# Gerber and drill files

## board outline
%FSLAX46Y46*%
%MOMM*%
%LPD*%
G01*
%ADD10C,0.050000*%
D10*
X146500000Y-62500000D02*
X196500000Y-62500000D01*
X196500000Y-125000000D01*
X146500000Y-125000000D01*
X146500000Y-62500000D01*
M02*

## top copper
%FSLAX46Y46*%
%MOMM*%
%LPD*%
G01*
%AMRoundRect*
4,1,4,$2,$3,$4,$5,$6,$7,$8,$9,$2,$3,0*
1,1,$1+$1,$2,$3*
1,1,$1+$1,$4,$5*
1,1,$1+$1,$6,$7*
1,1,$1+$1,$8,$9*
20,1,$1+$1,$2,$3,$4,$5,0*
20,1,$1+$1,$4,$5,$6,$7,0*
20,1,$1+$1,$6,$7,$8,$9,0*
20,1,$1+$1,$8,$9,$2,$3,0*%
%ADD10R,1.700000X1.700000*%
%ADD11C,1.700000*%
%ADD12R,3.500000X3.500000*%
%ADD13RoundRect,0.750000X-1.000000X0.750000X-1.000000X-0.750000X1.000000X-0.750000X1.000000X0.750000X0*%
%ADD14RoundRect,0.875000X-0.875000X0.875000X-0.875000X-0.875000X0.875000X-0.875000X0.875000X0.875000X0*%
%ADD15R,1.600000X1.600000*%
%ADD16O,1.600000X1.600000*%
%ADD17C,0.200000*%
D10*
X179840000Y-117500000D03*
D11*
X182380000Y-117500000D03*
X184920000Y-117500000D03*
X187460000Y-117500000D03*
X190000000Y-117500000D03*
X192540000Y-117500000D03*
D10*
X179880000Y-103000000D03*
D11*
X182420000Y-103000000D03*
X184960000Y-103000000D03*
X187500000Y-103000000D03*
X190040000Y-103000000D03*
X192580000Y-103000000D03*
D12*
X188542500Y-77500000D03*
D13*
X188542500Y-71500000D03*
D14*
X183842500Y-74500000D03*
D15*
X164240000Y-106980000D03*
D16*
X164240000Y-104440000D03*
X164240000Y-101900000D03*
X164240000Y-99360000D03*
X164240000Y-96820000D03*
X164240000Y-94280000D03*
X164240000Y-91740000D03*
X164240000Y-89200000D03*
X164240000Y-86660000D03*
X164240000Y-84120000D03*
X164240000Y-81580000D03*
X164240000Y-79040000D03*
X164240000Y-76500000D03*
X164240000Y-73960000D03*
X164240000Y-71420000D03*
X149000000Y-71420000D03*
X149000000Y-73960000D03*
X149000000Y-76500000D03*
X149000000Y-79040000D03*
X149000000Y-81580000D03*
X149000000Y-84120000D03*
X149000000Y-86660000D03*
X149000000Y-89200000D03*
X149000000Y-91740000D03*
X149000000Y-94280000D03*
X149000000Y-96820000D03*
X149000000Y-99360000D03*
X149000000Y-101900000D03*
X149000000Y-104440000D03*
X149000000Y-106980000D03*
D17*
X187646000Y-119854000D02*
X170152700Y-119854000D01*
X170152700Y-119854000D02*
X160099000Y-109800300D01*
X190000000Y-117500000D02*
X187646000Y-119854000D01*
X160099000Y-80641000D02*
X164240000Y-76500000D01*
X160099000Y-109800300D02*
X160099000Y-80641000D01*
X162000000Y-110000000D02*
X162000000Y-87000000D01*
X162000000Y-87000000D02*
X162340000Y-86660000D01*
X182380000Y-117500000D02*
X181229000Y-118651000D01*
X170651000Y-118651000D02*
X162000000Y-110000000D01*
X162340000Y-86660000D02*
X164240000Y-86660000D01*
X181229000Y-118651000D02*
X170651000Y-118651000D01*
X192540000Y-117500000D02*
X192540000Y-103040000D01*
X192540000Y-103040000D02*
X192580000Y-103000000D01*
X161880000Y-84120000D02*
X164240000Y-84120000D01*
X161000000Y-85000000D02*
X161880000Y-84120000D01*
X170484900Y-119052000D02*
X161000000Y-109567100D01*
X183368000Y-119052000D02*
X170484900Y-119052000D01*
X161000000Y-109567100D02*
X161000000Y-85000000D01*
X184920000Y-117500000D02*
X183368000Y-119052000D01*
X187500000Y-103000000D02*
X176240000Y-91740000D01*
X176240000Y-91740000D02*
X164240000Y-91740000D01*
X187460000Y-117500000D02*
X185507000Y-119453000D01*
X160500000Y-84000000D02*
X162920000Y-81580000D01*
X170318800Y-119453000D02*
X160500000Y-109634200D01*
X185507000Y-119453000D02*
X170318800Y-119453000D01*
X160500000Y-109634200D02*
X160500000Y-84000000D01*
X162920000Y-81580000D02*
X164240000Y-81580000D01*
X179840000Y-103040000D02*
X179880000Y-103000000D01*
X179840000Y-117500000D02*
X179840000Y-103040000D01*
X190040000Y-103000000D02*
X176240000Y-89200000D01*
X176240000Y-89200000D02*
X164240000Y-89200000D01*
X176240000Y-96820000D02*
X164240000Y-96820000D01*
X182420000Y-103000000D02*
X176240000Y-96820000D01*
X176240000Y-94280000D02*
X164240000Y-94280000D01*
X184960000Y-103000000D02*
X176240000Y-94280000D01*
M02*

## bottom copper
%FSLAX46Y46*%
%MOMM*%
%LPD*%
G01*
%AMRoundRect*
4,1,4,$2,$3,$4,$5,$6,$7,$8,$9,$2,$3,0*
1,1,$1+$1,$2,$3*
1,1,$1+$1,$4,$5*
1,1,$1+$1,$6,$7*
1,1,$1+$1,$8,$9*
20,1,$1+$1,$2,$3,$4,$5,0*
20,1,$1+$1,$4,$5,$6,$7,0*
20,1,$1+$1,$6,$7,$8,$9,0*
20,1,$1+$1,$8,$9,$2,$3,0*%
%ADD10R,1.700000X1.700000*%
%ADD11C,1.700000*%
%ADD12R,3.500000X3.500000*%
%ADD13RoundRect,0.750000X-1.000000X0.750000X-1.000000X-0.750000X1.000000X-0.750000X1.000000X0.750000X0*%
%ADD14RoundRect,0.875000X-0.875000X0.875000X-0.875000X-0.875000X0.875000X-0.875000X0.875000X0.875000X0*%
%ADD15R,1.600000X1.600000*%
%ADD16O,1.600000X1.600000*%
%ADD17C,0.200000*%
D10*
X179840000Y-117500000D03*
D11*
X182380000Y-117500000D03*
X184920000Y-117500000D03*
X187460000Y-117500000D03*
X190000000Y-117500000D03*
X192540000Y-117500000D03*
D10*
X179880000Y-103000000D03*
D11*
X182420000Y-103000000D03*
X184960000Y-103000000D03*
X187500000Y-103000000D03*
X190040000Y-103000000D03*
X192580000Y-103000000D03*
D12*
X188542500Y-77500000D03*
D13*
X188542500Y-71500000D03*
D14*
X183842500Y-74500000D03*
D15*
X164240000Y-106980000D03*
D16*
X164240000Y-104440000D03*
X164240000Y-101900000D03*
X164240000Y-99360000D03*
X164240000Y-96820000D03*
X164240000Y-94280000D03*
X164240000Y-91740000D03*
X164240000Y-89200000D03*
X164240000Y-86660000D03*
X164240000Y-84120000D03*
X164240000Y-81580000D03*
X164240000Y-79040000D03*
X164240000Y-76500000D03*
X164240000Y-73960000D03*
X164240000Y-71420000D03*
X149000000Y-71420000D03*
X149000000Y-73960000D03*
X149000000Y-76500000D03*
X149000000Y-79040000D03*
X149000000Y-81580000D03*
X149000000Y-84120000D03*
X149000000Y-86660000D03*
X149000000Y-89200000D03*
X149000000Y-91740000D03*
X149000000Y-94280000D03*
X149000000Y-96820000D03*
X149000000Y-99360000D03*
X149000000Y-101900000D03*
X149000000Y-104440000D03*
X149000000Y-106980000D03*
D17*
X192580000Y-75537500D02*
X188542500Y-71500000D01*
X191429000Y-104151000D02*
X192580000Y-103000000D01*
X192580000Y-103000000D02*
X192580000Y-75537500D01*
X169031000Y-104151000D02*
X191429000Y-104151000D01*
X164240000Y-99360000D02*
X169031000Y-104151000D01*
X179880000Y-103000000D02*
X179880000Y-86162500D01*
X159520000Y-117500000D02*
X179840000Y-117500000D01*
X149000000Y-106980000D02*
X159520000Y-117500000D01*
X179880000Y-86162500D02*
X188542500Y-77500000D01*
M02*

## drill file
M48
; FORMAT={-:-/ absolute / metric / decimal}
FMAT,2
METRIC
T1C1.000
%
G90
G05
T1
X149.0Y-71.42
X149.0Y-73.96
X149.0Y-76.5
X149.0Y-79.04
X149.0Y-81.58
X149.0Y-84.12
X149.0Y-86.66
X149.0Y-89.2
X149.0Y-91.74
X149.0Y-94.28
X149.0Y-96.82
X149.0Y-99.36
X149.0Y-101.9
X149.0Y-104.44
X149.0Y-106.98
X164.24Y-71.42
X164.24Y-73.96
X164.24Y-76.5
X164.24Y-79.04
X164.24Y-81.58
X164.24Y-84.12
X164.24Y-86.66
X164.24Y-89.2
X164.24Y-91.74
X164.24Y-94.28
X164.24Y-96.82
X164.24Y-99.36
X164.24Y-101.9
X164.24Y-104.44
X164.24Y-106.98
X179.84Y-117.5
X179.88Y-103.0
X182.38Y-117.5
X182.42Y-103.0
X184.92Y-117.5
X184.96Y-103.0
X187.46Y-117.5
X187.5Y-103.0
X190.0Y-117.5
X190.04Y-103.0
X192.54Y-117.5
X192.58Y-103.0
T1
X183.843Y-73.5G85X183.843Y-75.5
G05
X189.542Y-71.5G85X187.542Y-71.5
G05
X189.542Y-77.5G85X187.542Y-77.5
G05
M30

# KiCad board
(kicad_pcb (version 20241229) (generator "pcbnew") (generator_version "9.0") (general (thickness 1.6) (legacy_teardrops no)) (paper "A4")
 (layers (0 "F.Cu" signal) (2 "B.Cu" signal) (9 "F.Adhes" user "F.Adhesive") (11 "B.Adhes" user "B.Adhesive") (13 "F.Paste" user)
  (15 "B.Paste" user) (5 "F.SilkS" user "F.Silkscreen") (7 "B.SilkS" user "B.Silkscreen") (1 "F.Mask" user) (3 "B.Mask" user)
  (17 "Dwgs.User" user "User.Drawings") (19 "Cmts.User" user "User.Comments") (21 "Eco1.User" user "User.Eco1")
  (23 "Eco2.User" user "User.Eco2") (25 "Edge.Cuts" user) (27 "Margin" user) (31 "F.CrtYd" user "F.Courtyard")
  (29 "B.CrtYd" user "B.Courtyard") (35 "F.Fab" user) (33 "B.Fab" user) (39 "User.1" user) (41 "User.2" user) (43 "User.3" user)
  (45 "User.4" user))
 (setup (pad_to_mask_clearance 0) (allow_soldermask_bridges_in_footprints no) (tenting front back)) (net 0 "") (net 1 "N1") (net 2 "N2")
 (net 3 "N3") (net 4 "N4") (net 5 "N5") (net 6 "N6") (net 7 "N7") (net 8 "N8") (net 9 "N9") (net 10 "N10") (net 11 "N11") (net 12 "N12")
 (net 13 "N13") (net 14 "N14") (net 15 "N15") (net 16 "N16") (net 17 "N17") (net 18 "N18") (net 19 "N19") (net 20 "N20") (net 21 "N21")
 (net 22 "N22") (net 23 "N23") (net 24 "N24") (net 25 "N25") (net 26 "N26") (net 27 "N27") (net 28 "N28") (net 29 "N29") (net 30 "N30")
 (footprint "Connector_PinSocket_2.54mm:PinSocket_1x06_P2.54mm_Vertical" (layer "F.Cu") (at 179.84 117.5 90)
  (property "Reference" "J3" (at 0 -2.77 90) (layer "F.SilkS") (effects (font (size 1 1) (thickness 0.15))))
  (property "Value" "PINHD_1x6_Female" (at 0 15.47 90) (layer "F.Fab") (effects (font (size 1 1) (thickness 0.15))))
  (pad "1" thru_hole rect (at 0 0 90) (size 1.7 1.7) (drill 1) (layers "*.Cu" "*.Mask") (remove_unused_layers no) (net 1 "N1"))
  (pad "2" thru_hole circle (at 0 2.54 90) (size 1.7 1.7) (drill 1) (layers "*.Cu" "*.Mask") (remove_unused_layers no) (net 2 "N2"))
  (pad "3" thru_hole circle (at 0 5.08 90) (size 1.7 1.7) (drill 1) (layers "*.Cu" "*.Mask") (remove_unused_layers no) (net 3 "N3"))
  (pad "4" thru_hole circle (at 0 7.62 90) (size 1.7 1.7) (drill 1) (layers "*.Cu" "*.Mask") (remove_unused_layers no) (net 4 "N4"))
  (pad "5" thru_hole circle (at 0 10.16 90) (size 1.7 1.7) (drill 1) (layers "*.Cu" "*.Mask") (remove_unused_layers no) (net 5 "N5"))
  (pad "6" thru_hole circle (at 0 12.7 90) (size 1.7 1.7) (drill 1) (layers "*.Cu" "*.Mask") (remove_unused_layers no) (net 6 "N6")))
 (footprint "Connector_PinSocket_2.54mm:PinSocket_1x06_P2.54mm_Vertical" (layer "F.Cu") (at 179.88 103 90)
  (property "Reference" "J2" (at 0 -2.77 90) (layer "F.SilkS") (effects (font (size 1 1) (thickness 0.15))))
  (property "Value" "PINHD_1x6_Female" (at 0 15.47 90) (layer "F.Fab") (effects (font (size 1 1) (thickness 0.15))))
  (pad "1" thru_hole rect (at 0 0 90) (size 1.7 1.7) (drill 1) (layers "*.Cu" "*.Mask") (remove_unused_layers no) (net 1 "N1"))
  (pad "2" thru_hole circle (at 0 2.54 90) (size 1.7 1.7) (drill 1) (layers "*.Cu" "*.Mask") (remove_unused_layers no) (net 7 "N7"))
  (pad "3" thru_hole circle (at 0 5.08 90) (size 1.7 1.7) (drill 1) (layers "*.Cu" "*.Mask") (remove_unused_layers no) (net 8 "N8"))
  (pad "4" thru_hole circle (at 0 7.62 90) (size 1.7 1.7) (drill 1) (layers "*.Cu" "*.Mask") (remove_unused_layers no) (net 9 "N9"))
  (pad "5" thru_hole circle (at 0 10.16 90) (size 1.7 1.7) (drill 1) (layers "*.Cu" "*.Mask") (remove_unused_layers no) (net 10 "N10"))
  (pad "6" thru_hole circle (at 0 12.7 90) (size 1.7 1.7) (drill 1) (layers "*.Cu" "*.Mask") (remove_unused_layers no) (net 6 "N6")))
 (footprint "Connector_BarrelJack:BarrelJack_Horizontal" (layer "F.Cu") (at 188.5425 77.5 -90)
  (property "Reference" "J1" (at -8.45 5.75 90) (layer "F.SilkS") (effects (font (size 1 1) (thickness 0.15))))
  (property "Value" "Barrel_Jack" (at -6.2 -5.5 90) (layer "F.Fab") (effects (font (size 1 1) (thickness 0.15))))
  (pad "1" thru_hole rect (at 0 0 270) (size 3.5 3.5) (drill oval 1 3) (layers "*.Cu" "*.Mask") (remove_unused_layers no) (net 1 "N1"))
  (pad "2" thru_hole roundrect (at -6 0 270) (size 3 3.5) (drill oval 1 3) (layers "*.Cu" "*.Mask") (remove_unused_layers no)
   (roundrect_rratio 0.25) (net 6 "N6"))
  (pad "3" thru_hole roundrect (at -3 4.7 270) (size 3.5 3.5) (drill oval 3 1) (layers "*.Cu" "*.Mask") (remove_unused_layers no)
   (roundrect_rratio 0.25)))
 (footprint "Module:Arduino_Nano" (layer "F.Cu") (at 164.24 106.98 180)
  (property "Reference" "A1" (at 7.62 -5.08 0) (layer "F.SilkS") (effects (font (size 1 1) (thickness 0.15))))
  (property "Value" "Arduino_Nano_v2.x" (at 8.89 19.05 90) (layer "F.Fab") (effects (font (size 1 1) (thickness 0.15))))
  (pad "1" thru_hole rect (at 0 0 180) (size 1.6 1.6) (drill 1) (layers "*.Cu" "*.Mask") (remove_unused_layers no) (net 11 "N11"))
  (pad "2" thru_hole oval (at 0 2.54 180) (size 1.6 1.6) (drill 1) (layers "*.Cu" "*.Mask") (remove_unused_layers no) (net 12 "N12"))
  (pad "3" thru_hole oval (at 0 5.08 180) (size 1.6 1.6) (drill 1) (layers "*.Cu" "*.Mask") (remove_unused_layers no) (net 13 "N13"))
  (pad "4" thru_hole oval (at 0 7.62 180) (size 1.6 1.6) (drill 1) (layers "*.Cu" "*.Mask") (remove_unused_layers no) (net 6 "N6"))
  (pad "5" thru_hole oval (at 0 10.16 180) (size 1.6 1.6) (drill 1) (layers "*.Cu" "*.Mask") (remove_unused_layers no) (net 7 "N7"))
  (pad "6" thru_hole oval (at 0 12.7 180) (size 1.6 1.6) (drill 1) (layers "*.Cu" "*.Mask") (remove_unused_layers no) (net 8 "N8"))
  (pad "7" thru_hole oval (at 0 15.24 180) (size 1.6 1.6) (drill 1) (layers "*.Cu" "*.Mask") (remove_unused_layers no) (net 9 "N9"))
  (pad "8" thru_hole oval (at 0 17.78 180) (size 1.6 1.6) (drill 1) (layers "*.Cu" "*.Mask") (remove_unused_layers no) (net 10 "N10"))
  (pad "9" thru_hole oval (at 0 20.32 180) (size 1.6 1.6) (drill 1) (layers "*.Cu" "*.Mask") (remove_unused_layers no) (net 2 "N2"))
  (pad "10" thru_hole oval (at 0 22.86 180) (size 1.6 1.6) (drill 1) (layers "*.Cu" "*.Mask") (remove_unused_layers no) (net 3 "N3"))
  (pad "11" thru_hole oval (at 0 25.4 180) (size 1.6 1.6) (drill 1) (layers "*.Cu" "*.Mask") (remove_unused_layers no) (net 4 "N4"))
  (pad "12" thru_hole oval (at 0 27.94 180) (size 1.6 1.6) (drill 1) (layers "*.Cu" "*.Mask") (remove_unused_layers no) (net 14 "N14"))
  (pad "13" thru_hole oval (at 0 30.48 180) (size 1.6 1.6) (drill 1) (layers "*.Cu" "*.Mask") (remove_unused_layers no) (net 5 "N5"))
  (pad "14" thru_hole oval (at 0 33.02 180) (size 1.6 1.6) (drill 1) (layers "*.Cu" "*.Mask") (remove_unused_layers no) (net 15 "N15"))
  (pad "15" thru_hole oval (at 0 35.56 180) (size 1.6 1.6) (drill 1) (layers "*.Cu" "*.Mask") (remove_unused_layers no) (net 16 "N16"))
  (pad "16" thru_hole oval (at 15.24 35.56 180) (size 1.6 1.6) (drill 1) (layers "*.Cu" "*.Mask") (remove_unused_layers no) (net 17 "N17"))
  (pad "17" thru_hole oval (at 15.24 33.02 180) (size 1.6 1.6) (drill 1) (layers "*.Cu" "*.Mask") (remove_unused_layers no) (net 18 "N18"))
  (pad "18" thru_hole oval (at 15.24 30.48 180) (size 1.6 1.6) (drill 1) (layers "*.Cu" "*.Mask") (remove_unused_layers no) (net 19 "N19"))
  (pad "19" thru_hole oval (at 15.24 27.94 180) (size 1.6 1.6) (drill 1) (layers "*.Cu" "*.Mask") (remove_unused_layers no) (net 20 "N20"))
  (pad "20" thru_hole oval (at 15.24 25.4 180) (size 1.6 1.6) (drill 1) (layers "*.Cu" "*.Mask") (remove_unused_layers no) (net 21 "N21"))
  (pad "21" thru_hole oval (at 15.24 22.86 180) (size 1.6 1.6) (drill 1) (layers "*.Cu" "*.Mask") (remove_unused_layers no) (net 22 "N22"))
  (pad "22" thru_hole oval (at 15.24 20.32 180) (size 1.6 1.6) (drill 1) (layers "*.Cu" "*.Mask") (remove_unused_layers no) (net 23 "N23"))
  (pad "23" thru_hole oval (at 15.24 17.78 180) (size 1.6 1.6) (drill 1) (layers "*.Cu" "*.Mask") (remove_unused_layers no) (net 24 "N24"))
  (pad "24" thru_hole oval (at 15.24 15.24 180) (size 1.6 1.6) (drill 1) (layers "*.Cu" "*.Mask") (remove_unused_layers no) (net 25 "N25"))
  (pad "25" thru_hole oval (at 15.24 12.7 180) (size 1.6 1.6) (drill 1) (layers "*.Cu" "*.Mask") (remove_unused_layers no) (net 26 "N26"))
  (pad "26" thru_hole oval (at 15.24 10.16 180) (size 1.6 1.6) (drill 1) (layers "*.Cu" "*.Mask") (remove_unused_layers no) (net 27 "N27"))
  (pad "27" thru_hole oval (at 15.24 7.62 180) (size 1.6 1.6) (drill 1) (layers "*.Cu" "*.Mask") (remove_unused_layers no) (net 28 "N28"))
  (pad "28" thru_hole oval (at 15.24 5.08 180) (size 1.6 1.6) (drill 1) (layers "*.Cu" "*.Mask") (remove_unused_layers no) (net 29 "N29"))
  (pad "29" thru_hole oval (at 15.24 2.54 180) (size 1.6 1.6) (drill 1) (layers "*.Cu" "*.Mask") (remove_unused_layers no) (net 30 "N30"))
  (pad "30" thru_hole oval (at 15.24 0 180) (size 1.6 1.6) (drill 1) (layers "*.Cu" "*.Mask") (remove_unused_layers no) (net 1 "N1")))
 (gr_rect (start 146.5 62.5) (end 196.5 125) (stroke (width 0.05) (type default)) (fill no) (layer "Edge.Cuts"))
 (segment (start 187.646 119.854) (end 170.1527 119.854) (width 0.2) (layer "F.Cu") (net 5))
 (segment (start 170.1527 119.854) (end 160.099 109.8003) (width 0.2) (layer "F.Cu") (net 5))
 (segment (start 190 117.5) (end 187.646 119.854) (width 0.2) (layer "F.Cu") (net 5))
 (segment (start 160.099 80.641) (end 164.24 76.5) (width 0.2) (layer "F.Cu") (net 5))
 (segment (start 160.099 109.8003) (end 160.099 80.641) (width 0.2) (layer "F.Cu") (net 5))
 (segment (start 162 110) (end 162 87) (width 0.2) (layer "F.Cu") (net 2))
 (segment (start 162 87) (end 162.34 86.66) (width 0.2) (layer "F.Cu") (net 2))
 (segment (start 182.38 117.5) (end 181.229 118.651) (width 0.2) (layer "F.Cu") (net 2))
 (segment (start 170.651 118.651) (end 162 110) (width 0.2) (layer "F.Cu") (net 2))
 (segment (start 162.34 86.66) (end 164.24 86.66) (width 0.2) (layer "F.Cu") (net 2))
 (segment (start 181.229 118.651) (end 170.651 118.651) (width 0.2) (layer "F.Cu") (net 2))
 (segment (start 192.54 117.5) (end 192.54 103.04) (width 0.2) (layer "F.Cu") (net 6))
 (segment (start 192.54 103.04) (end 192.58 103) (width 0.2) (layer "F.Cu") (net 6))
 (segment (start 192.58 75.5375) (end 188.5425 71.5) (width 0.2) (layer "B.Cu") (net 6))
 (segment (start 191.429 104.151) (end 192.58 103) (width 0.2) (layer "B.Cu") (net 6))
 (segment (start 192.58 103) (end 192.58 75.5375) (width 0.2) (layer "B.Cu") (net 6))
 (segment (start 169.031 104.151) (end 191.429 104.151) (width 0.2) (layer "B.Cu") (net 6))
 (segment (start 164.24 99.36) (end 169.031 104.151) (width 0.2) (layer "B.Cu") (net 6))
 (segment (start 161.88 84.12) (end 164.24 84.12) (width 0.2) (layer "F.Cu") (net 3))
 (segment (start 161 85) (end 161.88 84.12) (width 0.2) (layer "F.Cu") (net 3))
 (segment (start 170.4849 119.052) (end 161 109.5671) (width 0.2) (layer "F.Cu") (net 3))
 (segment (start 183.368 119.052) (end 170.4849 119.052) (width 0.2) (layer "F.Cu") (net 3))
 (segment (start 161 109.5671) (end 161 85) (width 0.2) (layer "F.Cu") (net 3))
 (segment (start 184.92 117.5) (end 183.368 119.052) (width 0.2) (layer "F.Cu") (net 3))
 (segment (start 187.5 103) (end 176.24 91.74) (width 0.2) (layer "F.Cu") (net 9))
 (segment (start 176.24 91.74) (end 164.24 91.74) (width 0.2) (layer "F.Cu") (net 9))
 (segment (start 187.46 117.5) (end 185.507 119.453) (width 0.2) (layer "F.Cu") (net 4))
 (segment (start 160.5 84) (end 162.92 81.58) (width 0.2) (layer "F.Cu") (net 4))
 (segment (start 170.3188 119.453) (end 160.5 109.6342) (width 0.2) (layer "F.Cu") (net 4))
 (segment (start 185.507 119.453) (end 170.3188 119.453) (width 0.2) (layer "F.Cu") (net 4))
 (segment (start 160.5 109.6342) (end 160.5 84) (width 0.2) (layer "F.Cu") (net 4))
 (segment (start 162.92 81.58) (end 164.24 81.58) (width 0.2) (layer "F.Cu") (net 4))
 (segment (start 179.84 103.04) (end 179.88 103) (width 0.2) (layer "F.Cu") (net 1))
 (segment (start 179.84 117.5) (end 179.84 103.04) (width 0.2) (layer "F.Cu") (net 1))
 (segment (start 179.88 103) (end 179.88 86.1625) (width 0.2) (layer "B.Cu") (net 1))
 (segment (start 159.52 117.5) (end 179.84 117.5) (width 0.2) (layer "B.Cu") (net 1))
 (segment (start 149 106.98) (end 159.52 117.5) (width 0.2) (layer "B.Cu") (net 1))
 (segment (start 179.88 86.1625) (end 188.5425 77.5) (width 0.2) (layer "B.Cu") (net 1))
 (segment (start 190.04 103) (end 176.24 89.2) (width 0.2) (layer "F.Cu") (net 10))
 (segment (start 176.24 89.2) (end 164.24 89.2) (width 0.2) (layer "F.Cu") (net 10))
 (segment (start 176.24 96.82) (end 164.24 96.82) (width 0.2) (layer "F.Cu") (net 7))
 (segment (start 182.42 103) (end 176.24 96.82) (width 0.2) (layer "F.Cu") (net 7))
 (segment (start 176.24 94.28) (end 164.24 94.28) (width 0.2) (layer "F.Cu") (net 8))
 (segment (start 184.96 103) (end 176.24 94.28) (width 0.2) (layer "F.Cu") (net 8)))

